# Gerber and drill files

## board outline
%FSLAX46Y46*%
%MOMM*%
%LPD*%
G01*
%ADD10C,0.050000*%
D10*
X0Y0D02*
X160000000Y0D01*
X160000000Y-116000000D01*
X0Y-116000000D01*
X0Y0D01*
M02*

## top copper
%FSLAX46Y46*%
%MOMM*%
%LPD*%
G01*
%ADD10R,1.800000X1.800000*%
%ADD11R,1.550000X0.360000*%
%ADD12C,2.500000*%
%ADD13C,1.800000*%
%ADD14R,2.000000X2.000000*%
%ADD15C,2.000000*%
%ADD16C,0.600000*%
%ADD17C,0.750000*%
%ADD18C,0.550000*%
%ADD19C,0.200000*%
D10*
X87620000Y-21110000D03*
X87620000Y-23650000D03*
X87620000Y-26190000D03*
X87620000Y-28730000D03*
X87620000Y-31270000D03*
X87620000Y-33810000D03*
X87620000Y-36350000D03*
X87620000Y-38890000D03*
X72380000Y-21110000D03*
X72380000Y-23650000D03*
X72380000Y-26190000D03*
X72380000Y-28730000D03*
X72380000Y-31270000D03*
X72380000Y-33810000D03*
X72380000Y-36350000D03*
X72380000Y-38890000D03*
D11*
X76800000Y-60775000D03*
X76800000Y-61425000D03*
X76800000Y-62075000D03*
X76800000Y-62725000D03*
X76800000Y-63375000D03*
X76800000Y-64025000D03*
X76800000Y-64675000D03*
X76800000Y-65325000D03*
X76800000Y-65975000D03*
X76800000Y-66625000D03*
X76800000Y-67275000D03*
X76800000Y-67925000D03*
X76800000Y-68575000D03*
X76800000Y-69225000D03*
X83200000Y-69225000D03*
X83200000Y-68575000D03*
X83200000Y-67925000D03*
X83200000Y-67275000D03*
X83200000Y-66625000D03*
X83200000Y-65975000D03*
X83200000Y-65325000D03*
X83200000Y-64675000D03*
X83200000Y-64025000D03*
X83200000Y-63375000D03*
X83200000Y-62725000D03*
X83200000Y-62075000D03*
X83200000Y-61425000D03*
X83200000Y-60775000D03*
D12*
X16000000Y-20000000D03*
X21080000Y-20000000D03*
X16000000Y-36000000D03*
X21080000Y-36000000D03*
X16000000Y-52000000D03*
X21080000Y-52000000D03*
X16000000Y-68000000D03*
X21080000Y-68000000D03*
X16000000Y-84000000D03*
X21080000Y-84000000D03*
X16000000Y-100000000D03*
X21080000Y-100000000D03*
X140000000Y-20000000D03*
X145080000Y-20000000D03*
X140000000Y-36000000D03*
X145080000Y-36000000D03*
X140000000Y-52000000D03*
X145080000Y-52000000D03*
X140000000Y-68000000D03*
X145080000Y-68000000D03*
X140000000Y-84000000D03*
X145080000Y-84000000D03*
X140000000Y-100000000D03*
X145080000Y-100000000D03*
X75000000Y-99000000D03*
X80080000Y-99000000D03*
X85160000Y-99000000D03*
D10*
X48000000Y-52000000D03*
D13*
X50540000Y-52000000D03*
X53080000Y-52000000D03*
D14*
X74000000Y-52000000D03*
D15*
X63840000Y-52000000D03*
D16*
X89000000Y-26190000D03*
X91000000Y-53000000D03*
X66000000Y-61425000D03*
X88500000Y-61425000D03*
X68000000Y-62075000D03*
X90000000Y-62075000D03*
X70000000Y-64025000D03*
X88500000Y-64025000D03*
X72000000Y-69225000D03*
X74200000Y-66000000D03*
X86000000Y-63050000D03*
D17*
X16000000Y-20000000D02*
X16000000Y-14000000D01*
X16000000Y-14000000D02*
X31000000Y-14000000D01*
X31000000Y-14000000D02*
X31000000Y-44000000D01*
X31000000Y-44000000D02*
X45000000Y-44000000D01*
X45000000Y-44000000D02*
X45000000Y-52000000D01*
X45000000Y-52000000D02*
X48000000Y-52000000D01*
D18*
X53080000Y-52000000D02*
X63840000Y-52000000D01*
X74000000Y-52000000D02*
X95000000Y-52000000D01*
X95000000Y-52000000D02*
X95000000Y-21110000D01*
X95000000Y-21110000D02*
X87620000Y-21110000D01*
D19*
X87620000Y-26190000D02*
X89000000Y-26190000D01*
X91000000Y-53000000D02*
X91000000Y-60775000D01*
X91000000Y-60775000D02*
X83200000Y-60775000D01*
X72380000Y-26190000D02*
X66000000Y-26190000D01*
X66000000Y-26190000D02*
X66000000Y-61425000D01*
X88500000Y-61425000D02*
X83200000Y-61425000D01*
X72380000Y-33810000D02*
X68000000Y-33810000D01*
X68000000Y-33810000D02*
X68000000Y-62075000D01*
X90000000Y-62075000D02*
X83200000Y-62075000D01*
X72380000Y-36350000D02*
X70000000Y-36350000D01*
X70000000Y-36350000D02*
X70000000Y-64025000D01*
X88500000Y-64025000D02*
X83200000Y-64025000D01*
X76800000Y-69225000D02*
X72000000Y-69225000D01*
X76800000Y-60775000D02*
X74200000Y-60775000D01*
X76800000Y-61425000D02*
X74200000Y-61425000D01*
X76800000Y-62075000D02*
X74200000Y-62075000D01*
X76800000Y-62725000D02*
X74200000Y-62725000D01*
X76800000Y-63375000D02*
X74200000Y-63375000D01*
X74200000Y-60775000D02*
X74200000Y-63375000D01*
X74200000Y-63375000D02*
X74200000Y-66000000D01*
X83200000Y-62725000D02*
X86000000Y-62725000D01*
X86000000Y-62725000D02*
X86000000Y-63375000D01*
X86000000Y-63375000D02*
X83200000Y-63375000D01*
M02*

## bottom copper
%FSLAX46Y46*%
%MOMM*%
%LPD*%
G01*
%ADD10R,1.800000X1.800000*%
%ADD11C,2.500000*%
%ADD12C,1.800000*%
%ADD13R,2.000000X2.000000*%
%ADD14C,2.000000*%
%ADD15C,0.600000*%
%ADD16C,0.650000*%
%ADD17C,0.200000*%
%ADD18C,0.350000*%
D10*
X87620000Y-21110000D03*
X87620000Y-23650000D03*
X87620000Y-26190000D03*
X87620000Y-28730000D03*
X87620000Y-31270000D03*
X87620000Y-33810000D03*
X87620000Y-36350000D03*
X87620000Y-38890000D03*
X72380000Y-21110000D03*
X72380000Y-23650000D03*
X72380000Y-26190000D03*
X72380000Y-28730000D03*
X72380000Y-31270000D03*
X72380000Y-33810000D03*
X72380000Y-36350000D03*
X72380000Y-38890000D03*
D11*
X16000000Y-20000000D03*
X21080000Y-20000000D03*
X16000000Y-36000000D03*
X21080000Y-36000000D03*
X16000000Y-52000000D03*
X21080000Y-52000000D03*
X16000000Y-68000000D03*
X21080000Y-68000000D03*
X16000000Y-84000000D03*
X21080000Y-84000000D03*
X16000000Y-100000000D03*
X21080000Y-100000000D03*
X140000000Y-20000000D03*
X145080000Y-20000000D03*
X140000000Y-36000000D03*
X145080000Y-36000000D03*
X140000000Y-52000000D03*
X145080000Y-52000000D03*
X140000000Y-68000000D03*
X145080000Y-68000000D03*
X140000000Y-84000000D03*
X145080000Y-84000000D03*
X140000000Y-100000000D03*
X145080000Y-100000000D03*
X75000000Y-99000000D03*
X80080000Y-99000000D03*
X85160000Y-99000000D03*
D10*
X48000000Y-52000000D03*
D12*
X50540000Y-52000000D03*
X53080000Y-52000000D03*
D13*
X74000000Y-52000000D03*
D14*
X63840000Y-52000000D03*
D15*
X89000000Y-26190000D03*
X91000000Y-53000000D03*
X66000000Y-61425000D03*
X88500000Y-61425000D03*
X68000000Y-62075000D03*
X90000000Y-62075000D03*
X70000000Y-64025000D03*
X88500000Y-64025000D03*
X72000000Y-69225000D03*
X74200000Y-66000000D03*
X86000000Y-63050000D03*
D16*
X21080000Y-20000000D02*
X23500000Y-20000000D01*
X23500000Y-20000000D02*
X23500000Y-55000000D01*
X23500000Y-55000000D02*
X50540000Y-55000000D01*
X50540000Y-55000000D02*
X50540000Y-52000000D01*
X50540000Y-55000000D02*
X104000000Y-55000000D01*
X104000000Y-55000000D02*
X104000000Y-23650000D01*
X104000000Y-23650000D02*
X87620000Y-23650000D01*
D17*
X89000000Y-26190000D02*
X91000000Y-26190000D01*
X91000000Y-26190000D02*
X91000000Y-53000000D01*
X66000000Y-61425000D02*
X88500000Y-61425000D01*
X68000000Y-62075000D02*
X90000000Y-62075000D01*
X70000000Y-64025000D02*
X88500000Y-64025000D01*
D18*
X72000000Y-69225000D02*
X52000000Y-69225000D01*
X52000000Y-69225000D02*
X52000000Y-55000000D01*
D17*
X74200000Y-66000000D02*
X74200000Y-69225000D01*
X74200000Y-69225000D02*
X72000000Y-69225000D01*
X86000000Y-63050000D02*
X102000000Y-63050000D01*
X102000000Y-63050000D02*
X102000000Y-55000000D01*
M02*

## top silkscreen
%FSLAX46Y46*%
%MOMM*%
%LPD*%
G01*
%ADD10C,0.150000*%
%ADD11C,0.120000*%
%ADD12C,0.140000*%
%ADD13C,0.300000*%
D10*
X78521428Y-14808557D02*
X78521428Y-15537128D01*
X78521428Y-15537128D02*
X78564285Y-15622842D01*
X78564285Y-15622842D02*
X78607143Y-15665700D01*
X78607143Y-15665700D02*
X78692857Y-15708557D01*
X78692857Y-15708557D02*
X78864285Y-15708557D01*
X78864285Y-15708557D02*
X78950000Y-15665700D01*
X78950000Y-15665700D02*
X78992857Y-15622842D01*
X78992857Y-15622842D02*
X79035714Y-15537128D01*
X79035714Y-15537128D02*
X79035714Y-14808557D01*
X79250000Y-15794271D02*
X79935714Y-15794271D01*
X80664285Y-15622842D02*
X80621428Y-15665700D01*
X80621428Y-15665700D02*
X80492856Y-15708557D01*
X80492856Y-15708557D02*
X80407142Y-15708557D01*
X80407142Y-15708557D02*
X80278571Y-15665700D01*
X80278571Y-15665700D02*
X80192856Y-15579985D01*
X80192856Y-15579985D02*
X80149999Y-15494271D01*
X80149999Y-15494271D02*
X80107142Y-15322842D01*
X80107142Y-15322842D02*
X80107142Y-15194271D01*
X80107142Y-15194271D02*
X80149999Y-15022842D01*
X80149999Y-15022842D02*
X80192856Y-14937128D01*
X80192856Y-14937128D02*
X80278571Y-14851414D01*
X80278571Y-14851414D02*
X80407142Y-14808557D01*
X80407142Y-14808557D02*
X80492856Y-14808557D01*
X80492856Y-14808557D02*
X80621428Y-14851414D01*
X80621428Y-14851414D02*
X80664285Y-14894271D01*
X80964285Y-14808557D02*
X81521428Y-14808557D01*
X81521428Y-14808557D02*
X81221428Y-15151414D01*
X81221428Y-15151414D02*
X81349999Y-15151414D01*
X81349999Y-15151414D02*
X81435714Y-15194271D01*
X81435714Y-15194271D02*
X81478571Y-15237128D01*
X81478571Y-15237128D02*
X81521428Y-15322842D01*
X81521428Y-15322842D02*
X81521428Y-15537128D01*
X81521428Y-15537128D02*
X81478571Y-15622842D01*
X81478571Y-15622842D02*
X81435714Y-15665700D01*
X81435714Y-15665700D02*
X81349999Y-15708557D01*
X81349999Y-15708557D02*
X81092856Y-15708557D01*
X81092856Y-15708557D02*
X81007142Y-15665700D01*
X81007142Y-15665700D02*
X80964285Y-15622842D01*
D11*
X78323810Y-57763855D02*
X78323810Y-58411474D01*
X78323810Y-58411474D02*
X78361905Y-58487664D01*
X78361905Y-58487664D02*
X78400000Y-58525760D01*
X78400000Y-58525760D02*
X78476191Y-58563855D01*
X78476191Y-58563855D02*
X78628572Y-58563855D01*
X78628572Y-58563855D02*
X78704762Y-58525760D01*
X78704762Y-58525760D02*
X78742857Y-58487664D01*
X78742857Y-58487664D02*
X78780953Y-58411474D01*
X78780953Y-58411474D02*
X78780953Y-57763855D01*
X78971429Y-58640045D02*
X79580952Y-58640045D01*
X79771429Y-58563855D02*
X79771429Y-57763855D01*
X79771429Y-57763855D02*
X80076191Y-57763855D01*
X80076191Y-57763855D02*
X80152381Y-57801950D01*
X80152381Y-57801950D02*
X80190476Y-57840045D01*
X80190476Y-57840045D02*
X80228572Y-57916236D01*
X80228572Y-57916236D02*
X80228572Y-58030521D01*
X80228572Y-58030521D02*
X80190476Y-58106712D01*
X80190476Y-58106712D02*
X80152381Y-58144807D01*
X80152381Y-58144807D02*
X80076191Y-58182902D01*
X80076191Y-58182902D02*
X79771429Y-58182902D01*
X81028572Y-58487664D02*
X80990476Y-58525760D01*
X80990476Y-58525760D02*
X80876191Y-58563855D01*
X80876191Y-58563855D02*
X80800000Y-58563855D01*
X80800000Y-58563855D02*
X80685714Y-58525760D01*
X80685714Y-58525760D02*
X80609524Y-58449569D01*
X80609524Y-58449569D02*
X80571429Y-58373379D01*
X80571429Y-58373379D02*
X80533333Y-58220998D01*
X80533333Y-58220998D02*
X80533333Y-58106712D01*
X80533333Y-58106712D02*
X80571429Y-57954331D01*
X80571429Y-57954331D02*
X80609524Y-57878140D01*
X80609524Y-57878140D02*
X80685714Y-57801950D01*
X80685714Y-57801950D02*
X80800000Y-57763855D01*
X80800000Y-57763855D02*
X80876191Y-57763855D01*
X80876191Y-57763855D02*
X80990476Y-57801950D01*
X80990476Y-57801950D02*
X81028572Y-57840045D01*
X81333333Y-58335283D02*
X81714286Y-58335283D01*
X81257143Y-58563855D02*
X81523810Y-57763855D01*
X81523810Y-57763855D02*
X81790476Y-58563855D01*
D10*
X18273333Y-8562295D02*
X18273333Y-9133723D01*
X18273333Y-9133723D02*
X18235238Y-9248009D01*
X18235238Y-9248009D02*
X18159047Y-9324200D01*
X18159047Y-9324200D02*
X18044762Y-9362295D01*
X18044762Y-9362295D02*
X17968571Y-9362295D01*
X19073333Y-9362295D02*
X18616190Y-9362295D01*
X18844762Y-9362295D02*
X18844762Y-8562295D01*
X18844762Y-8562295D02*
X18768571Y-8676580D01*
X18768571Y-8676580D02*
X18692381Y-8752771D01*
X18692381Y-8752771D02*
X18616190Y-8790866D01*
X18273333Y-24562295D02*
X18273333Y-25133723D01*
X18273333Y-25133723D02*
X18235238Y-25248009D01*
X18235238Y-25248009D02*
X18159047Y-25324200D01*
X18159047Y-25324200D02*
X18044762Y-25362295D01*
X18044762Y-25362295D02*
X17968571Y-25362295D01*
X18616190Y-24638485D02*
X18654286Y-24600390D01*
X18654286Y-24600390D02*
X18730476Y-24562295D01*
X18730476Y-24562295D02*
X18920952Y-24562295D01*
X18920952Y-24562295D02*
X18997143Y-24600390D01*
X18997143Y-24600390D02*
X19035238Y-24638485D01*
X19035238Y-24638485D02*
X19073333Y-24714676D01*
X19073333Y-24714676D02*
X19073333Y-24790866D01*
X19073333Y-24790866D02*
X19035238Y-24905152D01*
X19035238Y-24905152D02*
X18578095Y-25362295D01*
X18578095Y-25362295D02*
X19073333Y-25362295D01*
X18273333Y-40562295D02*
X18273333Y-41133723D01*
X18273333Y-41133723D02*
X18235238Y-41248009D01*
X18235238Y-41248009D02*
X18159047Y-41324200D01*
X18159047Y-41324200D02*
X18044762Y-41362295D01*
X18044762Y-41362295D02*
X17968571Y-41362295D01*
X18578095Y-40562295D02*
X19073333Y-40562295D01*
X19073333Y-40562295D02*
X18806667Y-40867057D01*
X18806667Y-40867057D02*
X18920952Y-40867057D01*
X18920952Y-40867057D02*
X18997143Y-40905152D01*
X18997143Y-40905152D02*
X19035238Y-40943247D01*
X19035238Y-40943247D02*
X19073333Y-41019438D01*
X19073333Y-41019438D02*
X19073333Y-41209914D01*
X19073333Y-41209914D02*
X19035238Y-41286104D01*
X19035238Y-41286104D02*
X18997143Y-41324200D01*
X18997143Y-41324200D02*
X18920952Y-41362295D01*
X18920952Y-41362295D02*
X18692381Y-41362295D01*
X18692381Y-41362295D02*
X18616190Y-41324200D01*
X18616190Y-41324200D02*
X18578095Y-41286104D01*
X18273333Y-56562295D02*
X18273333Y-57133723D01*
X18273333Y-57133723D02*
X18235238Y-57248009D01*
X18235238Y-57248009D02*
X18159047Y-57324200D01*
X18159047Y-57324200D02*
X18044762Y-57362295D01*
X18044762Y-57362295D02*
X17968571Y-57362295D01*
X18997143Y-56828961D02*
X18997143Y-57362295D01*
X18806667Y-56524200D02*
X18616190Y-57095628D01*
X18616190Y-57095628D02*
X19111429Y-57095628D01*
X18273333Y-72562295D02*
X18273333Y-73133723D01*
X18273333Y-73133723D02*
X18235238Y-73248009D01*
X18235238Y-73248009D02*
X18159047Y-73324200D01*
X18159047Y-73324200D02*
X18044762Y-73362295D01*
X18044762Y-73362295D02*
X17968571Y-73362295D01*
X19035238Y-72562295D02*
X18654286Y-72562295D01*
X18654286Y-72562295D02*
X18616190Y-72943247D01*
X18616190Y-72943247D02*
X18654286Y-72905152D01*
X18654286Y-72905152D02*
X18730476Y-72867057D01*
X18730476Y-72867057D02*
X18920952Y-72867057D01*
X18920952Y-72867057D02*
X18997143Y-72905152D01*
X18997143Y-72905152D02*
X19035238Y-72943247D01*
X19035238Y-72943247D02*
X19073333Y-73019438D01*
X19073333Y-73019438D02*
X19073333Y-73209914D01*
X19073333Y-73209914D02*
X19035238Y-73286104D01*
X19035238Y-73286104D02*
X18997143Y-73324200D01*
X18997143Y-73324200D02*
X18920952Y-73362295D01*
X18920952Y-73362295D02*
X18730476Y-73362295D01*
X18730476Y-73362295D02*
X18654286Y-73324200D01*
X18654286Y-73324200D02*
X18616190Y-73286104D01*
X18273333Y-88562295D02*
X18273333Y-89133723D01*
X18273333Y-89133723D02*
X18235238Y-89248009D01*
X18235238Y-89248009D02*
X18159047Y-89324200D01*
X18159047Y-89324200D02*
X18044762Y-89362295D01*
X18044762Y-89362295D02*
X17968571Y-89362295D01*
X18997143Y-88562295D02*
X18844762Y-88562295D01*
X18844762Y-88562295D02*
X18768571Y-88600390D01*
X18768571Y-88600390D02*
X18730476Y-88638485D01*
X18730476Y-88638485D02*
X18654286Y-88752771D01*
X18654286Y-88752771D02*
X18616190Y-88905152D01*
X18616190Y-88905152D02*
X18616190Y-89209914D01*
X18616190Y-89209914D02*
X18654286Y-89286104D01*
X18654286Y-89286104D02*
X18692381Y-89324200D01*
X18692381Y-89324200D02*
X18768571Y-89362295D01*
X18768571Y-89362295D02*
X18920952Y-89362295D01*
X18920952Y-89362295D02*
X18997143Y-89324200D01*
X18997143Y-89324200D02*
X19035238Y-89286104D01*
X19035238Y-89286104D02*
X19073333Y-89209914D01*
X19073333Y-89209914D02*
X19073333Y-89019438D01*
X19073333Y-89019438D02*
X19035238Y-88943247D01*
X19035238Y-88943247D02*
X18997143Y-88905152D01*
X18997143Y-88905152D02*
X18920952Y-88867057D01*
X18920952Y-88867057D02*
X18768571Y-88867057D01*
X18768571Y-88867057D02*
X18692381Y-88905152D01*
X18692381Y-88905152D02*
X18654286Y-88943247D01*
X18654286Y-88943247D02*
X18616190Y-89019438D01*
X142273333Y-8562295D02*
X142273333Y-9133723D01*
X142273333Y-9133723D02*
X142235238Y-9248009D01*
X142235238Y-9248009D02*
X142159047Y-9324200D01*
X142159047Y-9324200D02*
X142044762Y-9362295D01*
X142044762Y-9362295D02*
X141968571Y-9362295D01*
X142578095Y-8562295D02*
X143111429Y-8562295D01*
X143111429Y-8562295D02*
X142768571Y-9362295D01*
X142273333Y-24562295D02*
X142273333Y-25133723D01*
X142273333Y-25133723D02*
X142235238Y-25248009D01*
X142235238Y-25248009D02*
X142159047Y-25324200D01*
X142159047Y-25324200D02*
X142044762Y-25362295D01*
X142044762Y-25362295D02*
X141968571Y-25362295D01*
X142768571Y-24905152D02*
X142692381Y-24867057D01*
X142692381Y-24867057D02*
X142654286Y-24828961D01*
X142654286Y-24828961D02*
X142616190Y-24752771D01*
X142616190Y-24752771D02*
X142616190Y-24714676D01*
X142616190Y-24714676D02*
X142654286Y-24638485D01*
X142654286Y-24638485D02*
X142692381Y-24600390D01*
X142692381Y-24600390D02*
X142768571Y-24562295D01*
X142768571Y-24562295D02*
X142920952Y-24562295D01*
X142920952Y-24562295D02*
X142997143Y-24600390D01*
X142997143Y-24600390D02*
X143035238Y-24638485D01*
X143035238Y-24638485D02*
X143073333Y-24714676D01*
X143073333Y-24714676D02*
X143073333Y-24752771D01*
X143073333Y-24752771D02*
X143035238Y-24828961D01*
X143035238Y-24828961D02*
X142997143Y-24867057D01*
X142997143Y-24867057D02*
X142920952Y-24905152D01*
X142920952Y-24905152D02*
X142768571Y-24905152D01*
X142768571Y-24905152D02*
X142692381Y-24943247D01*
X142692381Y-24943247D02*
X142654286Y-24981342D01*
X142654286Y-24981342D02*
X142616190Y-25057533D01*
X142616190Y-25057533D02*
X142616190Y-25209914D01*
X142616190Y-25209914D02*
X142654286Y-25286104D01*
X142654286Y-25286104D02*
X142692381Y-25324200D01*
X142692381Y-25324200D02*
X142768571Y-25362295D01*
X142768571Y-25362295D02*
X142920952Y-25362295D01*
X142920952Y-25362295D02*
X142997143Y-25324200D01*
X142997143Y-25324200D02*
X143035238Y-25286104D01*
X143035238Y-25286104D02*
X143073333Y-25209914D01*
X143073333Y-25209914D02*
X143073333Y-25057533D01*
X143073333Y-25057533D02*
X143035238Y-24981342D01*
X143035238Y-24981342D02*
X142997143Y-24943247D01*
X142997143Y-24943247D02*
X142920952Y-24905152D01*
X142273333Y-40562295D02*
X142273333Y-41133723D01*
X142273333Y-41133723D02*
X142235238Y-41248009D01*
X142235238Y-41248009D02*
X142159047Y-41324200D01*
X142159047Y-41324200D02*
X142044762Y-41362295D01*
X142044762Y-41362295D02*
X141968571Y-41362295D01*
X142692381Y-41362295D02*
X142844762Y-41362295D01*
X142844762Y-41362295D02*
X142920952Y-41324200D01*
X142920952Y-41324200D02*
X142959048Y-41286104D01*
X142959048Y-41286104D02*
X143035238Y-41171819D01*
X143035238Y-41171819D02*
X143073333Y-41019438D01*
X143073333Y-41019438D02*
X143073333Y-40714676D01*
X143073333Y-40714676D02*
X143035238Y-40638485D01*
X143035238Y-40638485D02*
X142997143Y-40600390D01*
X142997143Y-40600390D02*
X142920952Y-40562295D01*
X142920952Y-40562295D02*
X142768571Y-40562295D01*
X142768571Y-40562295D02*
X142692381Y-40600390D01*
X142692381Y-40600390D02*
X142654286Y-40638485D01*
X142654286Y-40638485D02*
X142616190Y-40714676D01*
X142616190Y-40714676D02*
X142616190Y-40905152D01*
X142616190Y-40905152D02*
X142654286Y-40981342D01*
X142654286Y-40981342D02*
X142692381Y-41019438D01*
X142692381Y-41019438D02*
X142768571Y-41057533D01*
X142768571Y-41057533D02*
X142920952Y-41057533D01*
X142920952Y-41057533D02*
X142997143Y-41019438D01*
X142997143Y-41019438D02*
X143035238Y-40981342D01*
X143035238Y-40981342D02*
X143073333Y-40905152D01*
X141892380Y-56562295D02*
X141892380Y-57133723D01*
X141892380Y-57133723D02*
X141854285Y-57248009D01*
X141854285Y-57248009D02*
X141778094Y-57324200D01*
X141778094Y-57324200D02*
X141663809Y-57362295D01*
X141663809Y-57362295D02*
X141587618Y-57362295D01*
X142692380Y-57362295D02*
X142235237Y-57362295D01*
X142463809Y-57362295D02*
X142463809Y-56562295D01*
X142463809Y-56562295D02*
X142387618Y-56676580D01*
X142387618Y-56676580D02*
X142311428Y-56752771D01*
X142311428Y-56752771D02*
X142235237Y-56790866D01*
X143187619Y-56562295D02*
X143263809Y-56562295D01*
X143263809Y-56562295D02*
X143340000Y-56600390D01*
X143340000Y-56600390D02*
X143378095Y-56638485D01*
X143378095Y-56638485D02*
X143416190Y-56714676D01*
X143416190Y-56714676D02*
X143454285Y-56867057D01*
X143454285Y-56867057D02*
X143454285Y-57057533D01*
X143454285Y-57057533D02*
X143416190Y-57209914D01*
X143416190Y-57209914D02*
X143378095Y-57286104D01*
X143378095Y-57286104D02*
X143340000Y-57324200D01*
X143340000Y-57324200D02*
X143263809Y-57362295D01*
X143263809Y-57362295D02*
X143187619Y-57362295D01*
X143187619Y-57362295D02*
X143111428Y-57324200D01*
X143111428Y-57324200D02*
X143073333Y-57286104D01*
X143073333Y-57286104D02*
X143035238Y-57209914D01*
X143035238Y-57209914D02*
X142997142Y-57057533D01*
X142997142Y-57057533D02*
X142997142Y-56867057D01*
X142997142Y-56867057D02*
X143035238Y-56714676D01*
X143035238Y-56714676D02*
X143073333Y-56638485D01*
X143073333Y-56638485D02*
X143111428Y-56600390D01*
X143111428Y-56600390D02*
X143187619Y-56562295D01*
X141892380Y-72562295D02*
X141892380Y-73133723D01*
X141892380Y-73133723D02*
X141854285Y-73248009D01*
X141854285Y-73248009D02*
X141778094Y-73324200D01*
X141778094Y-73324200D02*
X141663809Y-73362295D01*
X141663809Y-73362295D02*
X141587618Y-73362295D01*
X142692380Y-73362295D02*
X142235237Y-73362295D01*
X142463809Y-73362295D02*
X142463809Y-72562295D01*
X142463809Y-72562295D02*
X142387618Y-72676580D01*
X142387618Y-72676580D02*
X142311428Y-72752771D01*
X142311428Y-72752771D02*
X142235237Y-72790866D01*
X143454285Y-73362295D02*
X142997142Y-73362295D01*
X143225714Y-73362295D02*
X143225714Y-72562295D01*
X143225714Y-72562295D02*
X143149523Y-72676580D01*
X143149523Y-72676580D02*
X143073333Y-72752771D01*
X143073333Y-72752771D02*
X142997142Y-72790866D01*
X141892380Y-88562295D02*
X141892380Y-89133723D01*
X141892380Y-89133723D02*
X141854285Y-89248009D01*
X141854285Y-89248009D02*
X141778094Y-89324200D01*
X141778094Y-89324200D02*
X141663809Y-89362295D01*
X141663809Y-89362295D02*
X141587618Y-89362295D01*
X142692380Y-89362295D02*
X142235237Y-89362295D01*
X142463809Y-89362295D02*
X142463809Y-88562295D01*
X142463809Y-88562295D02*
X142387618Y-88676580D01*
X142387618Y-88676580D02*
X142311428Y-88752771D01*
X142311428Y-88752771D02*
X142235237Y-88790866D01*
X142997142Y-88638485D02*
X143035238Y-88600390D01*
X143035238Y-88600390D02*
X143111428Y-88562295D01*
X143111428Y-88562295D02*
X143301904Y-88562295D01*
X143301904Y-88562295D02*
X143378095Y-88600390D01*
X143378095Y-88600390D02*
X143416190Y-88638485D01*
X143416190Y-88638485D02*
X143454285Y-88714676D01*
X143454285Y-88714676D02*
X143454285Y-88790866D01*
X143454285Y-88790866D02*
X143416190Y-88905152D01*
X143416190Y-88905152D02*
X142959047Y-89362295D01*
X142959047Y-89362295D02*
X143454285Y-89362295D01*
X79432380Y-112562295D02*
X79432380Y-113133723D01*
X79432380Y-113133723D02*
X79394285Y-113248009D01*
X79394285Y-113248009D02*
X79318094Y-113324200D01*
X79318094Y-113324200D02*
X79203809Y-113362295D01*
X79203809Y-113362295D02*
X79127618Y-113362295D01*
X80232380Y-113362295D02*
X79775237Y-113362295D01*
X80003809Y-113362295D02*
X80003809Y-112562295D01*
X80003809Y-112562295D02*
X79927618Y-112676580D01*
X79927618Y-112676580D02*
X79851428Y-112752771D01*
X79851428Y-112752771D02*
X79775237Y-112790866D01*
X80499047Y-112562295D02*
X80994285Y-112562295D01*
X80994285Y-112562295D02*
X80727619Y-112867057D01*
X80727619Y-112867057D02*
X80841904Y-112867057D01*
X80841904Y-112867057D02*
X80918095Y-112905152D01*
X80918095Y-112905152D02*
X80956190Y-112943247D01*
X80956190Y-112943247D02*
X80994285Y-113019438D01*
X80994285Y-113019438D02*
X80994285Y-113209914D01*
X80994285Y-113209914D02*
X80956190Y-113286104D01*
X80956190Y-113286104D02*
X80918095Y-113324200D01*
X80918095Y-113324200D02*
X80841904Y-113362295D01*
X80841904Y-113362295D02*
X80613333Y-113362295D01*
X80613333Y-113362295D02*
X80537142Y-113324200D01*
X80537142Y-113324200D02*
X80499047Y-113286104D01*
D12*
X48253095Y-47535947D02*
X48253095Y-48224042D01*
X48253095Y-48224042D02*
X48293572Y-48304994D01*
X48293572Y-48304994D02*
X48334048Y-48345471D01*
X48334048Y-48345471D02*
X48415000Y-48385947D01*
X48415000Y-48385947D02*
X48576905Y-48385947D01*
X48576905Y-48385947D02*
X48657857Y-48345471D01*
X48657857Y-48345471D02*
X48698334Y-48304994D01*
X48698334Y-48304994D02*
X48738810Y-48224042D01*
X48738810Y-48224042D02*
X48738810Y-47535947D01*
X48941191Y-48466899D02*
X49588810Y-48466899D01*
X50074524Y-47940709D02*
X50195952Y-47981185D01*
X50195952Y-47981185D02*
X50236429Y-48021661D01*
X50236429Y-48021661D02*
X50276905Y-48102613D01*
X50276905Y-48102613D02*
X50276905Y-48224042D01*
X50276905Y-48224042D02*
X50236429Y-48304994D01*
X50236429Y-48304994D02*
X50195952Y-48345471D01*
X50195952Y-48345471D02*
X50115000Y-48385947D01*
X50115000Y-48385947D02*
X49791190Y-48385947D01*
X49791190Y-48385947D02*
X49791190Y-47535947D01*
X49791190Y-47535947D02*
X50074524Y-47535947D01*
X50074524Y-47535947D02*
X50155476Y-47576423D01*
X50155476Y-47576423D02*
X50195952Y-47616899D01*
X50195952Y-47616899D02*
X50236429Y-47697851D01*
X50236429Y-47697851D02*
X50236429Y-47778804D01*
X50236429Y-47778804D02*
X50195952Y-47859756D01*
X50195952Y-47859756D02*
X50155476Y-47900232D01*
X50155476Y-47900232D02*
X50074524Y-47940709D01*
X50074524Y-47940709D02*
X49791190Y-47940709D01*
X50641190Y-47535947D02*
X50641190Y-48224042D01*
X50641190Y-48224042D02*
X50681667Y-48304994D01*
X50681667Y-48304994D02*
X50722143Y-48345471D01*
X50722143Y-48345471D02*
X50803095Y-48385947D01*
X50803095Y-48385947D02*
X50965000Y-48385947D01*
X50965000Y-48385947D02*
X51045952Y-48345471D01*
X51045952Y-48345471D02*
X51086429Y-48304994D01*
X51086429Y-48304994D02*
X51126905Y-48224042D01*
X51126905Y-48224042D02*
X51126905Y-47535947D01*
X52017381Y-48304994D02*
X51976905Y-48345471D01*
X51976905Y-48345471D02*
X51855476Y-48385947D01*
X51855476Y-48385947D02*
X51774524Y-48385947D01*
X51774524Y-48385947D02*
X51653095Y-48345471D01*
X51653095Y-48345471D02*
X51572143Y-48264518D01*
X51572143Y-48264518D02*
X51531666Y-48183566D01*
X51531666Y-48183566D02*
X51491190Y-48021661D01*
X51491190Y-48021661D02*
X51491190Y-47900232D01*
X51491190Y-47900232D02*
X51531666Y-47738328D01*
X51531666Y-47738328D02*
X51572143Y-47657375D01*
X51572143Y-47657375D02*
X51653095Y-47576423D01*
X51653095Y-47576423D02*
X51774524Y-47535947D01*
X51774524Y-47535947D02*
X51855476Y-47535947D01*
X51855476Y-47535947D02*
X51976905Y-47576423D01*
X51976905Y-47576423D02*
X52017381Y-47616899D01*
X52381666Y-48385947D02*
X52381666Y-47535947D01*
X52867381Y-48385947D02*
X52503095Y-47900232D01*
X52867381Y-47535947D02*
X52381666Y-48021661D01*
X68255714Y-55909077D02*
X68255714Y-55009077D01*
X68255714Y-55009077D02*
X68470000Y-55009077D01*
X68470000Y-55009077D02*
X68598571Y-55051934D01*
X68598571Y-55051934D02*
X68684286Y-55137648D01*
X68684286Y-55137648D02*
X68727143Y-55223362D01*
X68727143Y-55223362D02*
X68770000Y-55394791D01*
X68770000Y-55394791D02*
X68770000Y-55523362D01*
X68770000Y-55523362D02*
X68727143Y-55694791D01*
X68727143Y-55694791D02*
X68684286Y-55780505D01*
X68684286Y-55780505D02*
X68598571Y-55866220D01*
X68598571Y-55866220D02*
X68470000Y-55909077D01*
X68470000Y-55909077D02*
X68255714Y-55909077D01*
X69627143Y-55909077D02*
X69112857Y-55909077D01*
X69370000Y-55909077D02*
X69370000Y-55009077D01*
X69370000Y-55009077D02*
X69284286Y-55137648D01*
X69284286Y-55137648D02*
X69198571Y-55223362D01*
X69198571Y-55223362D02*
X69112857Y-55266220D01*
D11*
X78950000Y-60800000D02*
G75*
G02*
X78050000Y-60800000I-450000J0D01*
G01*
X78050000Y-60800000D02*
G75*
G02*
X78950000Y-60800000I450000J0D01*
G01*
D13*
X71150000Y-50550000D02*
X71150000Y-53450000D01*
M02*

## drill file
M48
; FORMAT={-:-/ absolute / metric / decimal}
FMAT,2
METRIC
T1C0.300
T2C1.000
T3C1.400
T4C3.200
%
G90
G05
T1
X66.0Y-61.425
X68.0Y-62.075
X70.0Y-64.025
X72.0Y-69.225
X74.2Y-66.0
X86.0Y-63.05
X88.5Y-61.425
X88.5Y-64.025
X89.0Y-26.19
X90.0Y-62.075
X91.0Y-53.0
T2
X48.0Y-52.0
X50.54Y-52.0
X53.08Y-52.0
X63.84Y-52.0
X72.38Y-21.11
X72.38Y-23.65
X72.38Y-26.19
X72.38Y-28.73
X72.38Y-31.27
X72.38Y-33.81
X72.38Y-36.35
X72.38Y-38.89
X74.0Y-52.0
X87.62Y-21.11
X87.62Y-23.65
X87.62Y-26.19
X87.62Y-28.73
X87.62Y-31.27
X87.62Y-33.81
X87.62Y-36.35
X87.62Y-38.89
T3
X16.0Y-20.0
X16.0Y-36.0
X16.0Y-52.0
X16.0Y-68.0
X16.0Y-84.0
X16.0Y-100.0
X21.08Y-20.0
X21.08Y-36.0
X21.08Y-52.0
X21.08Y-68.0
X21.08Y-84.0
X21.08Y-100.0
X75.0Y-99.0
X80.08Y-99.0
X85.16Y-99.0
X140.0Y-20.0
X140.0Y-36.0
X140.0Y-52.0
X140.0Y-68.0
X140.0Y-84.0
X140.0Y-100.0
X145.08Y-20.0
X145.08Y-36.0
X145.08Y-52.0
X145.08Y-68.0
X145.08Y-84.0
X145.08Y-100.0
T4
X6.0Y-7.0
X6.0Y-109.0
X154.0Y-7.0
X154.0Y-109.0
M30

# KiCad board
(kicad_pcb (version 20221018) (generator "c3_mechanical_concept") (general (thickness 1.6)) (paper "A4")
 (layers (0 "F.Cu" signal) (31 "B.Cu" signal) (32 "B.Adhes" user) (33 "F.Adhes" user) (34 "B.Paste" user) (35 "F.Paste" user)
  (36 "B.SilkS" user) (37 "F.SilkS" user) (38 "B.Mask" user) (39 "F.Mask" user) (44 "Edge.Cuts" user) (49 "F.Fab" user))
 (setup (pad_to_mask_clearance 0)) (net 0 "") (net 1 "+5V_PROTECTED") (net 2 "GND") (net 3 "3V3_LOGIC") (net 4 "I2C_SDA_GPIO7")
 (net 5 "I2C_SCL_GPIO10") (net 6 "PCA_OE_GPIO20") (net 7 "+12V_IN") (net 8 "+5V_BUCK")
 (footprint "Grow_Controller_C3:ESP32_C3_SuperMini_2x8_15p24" (layer "F.Cu") (at 80 30)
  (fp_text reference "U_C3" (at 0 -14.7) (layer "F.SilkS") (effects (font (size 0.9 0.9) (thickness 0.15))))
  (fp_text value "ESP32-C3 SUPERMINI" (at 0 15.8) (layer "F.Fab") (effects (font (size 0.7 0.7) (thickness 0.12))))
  (pad "1" thru_hole rect (at 7.62 -8.89) (size 1.8 1.8) (drill 1.0) (layers "*.Cu" "*.Mask") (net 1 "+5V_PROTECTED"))
  (pad "2" thru_hole rect (at 7.62 -6.35) (size 1.8 1.8) (drill 1.0) (layers "*.Cu" "*.Mask") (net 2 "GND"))
  (pad "3" thru_hole rect (at 7.62 -3.81) (size 1.8 1.8) (drill 1.0) (layers "*.Cu" "*.Mask") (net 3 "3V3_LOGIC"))
  (pad "4" thru_hole rect (at 7.62 -1.27) (size 1.8 1.8) (drill 1.0) (layers "*.Cu" "*.Mask"))
  (pad "5" thru_hole rect (at 7.62 1.27) (size 1.8 1.8) (drill 1.0) (layers "*.Cu" "*.Mask"))
  (pad "6" thru_hole rect (at 7.62 3.81) (size 1.8 1.8) (drill 1.0) (layers "*.Cu" "*.Mask"))
  (pad "7" thru_hole rect (at 7.62 6.35) (size 1.8 1.8) (drill 1.0) (layers "*.Cu" "*.Mask"))
  (pad "8" thru_hole rect (at 7.62 8.89) (size 1.8 1.8) (drill 1.0) (layers "*.Cu" "*.Mask"))
  (pad "9" thru_hole rect (at -7.62 -8.89) (size 1.8 1.8) (drill 1.0) (layers "*.Cu" "*.Mask"))
  (pad "10" thru_hole rect (at -7.62 -6.35) (size 1.8 1.8) (drill 1.0) (layers "*.Cu" "*.Mask"))
  (pad "11" thru_hole rect (at -7.62 -3.81) (size 1.8 1.8) (drill 1.0) (layers "*.Cu" "*.Mask") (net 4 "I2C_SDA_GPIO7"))
  (pad "12" thru_hole rect (at -7.62 -1.27) (size 1.8 1.8) (drill 1.0) (layers "*.Cu" "*.Mask"))
  (pad "13" thru_hole rect (at -7.62 1.27) (size 1.8 1.8) (drill 1.0) (layers "*.Cu" "*.Mask"))
  (pad "14" thru_hole rect (at -7.62 3.81) (size 1.8 1.8) (drill 1.0) (layers "*.Cu" "*.Mask") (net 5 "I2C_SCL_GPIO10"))
  (pad "15" thru_hole rect (at -7.62 6.35) (size 1.8 1.8) (drill 1.0) (layers "*.Cu" "*.Mask") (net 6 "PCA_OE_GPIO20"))
  (pad "16" thru_hole rect (at -7.62 8.89) (size 1.8 1.8) (drill 1.0) (layers "*.Cu" "*.Mask")))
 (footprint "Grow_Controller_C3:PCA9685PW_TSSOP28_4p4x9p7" (layer "F.Cu") (at 80 65)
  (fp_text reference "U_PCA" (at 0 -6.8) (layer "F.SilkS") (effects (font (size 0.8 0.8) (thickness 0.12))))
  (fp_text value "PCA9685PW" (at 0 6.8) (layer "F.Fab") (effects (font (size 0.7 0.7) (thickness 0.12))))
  (fp_circle (center -1.5 -4.2) (end -1.05 -4.2) (stroke (width 0.12) (type solid)) (fill none) (layer "F.SilkS"))
  (pad "1" smd rect (at -3.200 -4.225) (size 1.55 0.36) (layers "F.Cu" "F.Paste" "F.Mask") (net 2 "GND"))
  (pad "2" smd rect (at -3.200 -3.575) (size 1.55 0.36) (layers "F.Cu" "F.Paste" "F.Mask") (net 2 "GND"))
  (pad "3" smd rect (at -3.200 -2.925) (size 1.55 0.36) (layers "F.Cu" "F.Paste" "F.Mask") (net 2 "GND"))
  (pad "4" smd rect (at -3.200 -2.275) (size 1.55 0.36) (layers "F.Cu" "F.Paste" "F.Mask") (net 2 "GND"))
  (pad "5" smd rect (at -3.200 -1.625) (size 1.55 0.36) (layers "F.Cu" "F.Paste" "F.Mask") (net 2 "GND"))
  (pad "6" smd rect (at -3.200 -0.975) (size 1.55 0.36) (layers "F.Cu" "F.Paste" "F.Mask"))
  (pad "7" smd rect (at -3.200 -0.325) (size 1.55 0.36) (layers "F.Cu" "F.Paste" "F.Mask"))
  (pad "8" smd rect (at -3.200 0.325) (size 1.55 0.36) (layers "F.Cu" "F.Paste" "F.Mask"))
  (pad "9" smd rect (at -3.200 0.975) (size 1.55 0.36) (layers "F.Cu" "F.Paste" "F.Mask"))
  (pad "10" smd rect (at -3.200 1.625) (size 1.55 0.36) (layers "F.Cu" "F.Paste" "F.Mask"))
  (pad "11" smd rect (at -3.200 2.275) (size 1.55 0.36) (layers "F.Cu" "F.Paste" "F.Mask"))
  (pad "12" smd rect (at -3.200 2.925) (size 1.55 0.36) (layers "F.Cu" "F.Paste" "F.Mask"))
  (pad "13" smd rect (at -3.200 3.575) (size 1.55 0.36) (layers "F.Cu" "F.Paste" "F.Mask"))
  (pad "14" smd rect (at -3.200 4.225) (size 1.55 0.36) (layers "F.Cu" "F.Paste" "F.Mask") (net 2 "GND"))
  (pad "15" smd rect (at 3.200 4.225) (size 1.55 0.36) (layers "F.Cu" "F.Paste" "F.Mask"))
  (pad "16" smd rect (at 3.200 3.575) (size 1.55 0.36) (layers "F.Cu" "F.Paste" "F.Mask"))
  (pad "17" smd rect (at 3.200 2.925) (size 1.55 0.36) (layers "F.Cu" "F.Paste" "F.Mask"))
  (pad "18" smd rect (at 3.200 2.275) (size 1.55 0.36) (layers "F.Cu" "F.Paste" "F.Mask"))
  (pad "19" smd rect (at 3.200 1.625) (size 1.55 0.36) (layers "F.Cu" "F.Paste" "F.Mask"))
  (pad "20" smd rect (at 3.200 0.975) (size 1.55 0.36) (layers "F.Cu" "F.Paste" "F.Mask"))
  (pad "21" smd rect (at 3.200 0.325) (size 1.55 0.36) (layers "F.Cu" "F.Paste" "F.Mask"))
  (pad "22" smd rect (at 3.200 -0.325) (size 1.55 0.36) (layers "F.Cu" "F.Paste" "F.Mask"))
  (pad "23" smd rect (at 3.200 -0.975) (size 1.55 0.36) (layers "F.Cu" "F.Paste" "F.Mask") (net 6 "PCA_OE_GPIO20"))
  (pad "24" smd rect (at 3.200 -1.625) (size 1.55 0.36) (layers "F.Cu" "F.Paste" "F.Mask") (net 2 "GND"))
  (pad "25" smd rect (at 3.200 -2.275) (size 1.55 0.36) (layers "F.Cu" "F.Paste" "F.Mask") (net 2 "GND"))
  (pad "26" smd rect (at 3.200 -2.925) (size 1.55 0.36) (layers "F.Cu" "F.Paste" "F.Mask") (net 5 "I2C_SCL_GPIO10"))
  (pad "27" smd rect (at 3.200 -3.575) (size 1.55 0.36) (layers "F.Cu" "F.Paste" "F.Mask") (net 4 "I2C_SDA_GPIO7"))
  (pad "28" smd rect (at 3.200 -4.225) (size 1.55 0.36) (layers "F.Cu" "F.Paste" "F.Mask") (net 3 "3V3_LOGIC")))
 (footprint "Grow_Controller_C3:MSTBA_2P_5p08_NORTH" (layer "F.Cu") (at 16 20)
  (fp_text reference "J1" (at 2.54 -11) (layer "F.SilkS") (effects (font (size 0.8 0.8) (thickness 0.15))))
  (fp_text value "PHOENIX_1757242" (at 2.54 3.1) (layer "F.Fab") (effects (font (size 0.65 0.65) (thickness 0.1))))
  (pad "1" thru_hole circle (at 0.00 0) (size 2.5 2.5) (drill 1.4) (layers "*.Cu" "*.Mask") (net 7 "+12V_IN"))
  (pad "2" thru_hole circle (at 5.08 0) (size 2.5 2.5) (drill 1.4) (layers "*.Cu" "*.Mask") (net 2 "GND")))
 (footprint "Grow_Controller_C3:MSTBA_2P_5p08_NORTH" (layer "F.Cu") (at 16 36)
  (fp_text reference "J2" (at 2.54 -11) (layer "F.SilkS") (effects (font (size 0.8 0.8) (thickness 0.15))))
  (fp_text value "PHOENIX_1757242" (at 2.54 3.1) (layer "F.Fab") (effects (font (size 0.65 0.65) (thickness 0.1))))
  (pad "1" thru_hole circle (at 0.00 0) (size 2.5 2.5) (drill 1.4) (layers "*.Cu" "*.Mask"))
  (pad "2" thru_hole circle (at 5.08 0) (size 2.5 2.5) (drill 1.4) (layers "*.Cu" "*.Mask")))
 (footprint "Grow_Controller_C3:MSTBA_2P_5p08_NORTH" (layer "F.Cu") (at 16 52)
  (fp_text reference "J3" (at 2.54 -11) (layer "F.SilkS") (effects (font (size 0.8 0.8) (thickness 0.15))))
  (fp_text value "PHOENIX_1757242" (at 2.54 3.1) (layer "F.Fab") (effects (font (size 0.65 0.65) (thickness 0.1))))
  (pad "1" thru_hole circle (at 0.00 0) (size 2.5 2.5) (drill 1.4) (layers "*.Cu" "*.Mask"))
  (pad "2" thru_hole circle (at 5.08 0) (size 2.5 2.5) (drill 1.4) (layers "*.Cu" "*.Mask")))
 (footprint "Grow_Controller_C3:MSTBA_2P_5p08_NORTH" (layer "F.Cu") (at 16 68)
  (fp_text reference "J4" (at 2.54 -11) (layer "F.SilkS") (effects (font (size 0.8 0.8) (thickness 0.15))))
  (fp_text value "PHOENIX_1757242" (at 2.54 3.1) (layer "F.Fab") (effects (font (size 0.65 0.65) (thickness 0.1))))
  (pad "1" thru_hole circle (at 0.00 0) (size 2.5 2.5) (drill 1.4) (layers "*.Cu" "*.Mask"))
  (pad "2" thru_hole circle (at 5.08 0) (size 2.5 2.5) (drill 1.4) (layers "*.Cu" "*.Mask")))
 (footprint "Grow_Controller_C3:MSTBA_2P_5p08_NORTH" (layer "F.Cu") (at 16 84)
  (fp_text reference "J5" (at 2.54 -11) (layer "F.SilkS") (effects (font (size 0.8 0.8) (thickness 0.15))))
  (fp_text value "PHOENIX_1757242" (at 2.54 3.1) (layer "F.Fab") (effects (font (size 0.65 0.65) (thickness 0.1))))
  (pad "1" thru_hole circle (at 0.00 0) (size 2.5 2.5) (drill 1.4) (layers "*.Cu" "*.Mask"))
  (pad "2" thru_hole circle (at 5.08 0) (size 2.5 2.5) (drill 1.4) (layers "*.Cu" "*.Mask")))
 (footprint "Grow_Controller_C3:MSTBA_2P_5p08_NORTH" (layer "F.Cu") (at 16 100)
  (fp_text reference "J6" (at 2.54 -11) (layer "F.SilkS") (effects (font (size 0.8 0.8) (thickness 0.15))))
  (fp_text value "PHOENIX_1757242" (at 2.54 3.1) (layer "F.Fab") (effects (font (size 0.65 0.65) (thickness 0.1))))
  (pad "1" thru_hole circle (at 0.00 0) (size 2.5 2.5) (drill 1.4) (layers "*.Cu" "*.Mask"))
  (pad "2" thru_hole circle (at 5.08 0) (size 2.5 2.5) (drill 1.4) (layers "*.Cu" "*.Mask")))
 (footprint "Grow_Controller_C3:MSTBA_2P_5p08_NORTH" (layer "F.Cu") (at 140 20)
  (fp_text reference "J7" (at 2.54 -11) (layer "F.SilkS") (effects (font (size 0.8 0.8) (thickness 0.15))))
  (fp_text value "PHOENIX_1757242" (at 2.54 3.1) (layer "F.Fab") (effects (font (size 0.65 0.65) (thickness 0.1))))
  (pad "1" thru_hole circle (at 0.00 0) (size 2.5 2.5) (drill 1.4) (layers "*.Cu" "*.Mask"))
  (pad "2" thru_hole circle (at 5.08 0) (size 2.5 2.5) (drill 1.4) (layers "*.Cu" "*.Mask")))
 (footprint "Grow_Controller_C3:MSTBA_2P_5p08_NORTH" (layer "F.Cu") (at 140 36)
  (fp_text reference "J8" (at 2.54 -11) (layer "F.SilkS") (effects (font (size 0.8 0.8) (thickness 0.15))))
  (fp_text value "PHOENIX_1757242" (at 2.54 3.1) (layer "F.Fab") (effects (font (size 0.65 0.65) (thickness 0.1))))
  (pad "1" thru_hole circle (at 0.00 0) (size 2.5 2.5) (drill 1.4) (layers "*.Cu" "*.Mask"))
  (pad "2" thru_hole circle (at 5.08 0) (size 2.5 2.5) (drill 1.4) (layers "*.Cu" "*.Mask")))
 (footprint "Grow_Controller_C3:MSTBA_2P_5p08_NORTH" (layer "F.Cu") (at 140 52)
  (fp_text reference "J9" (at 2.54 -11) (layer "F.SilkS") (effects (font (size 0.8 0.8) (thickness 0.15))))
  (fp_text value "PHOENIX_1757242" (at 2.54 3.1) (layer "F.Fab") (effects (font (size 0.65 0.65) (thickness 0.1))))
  (pad "1" thru_hole circle (at 0.00 0) (size 2.5 2.5) (drill 1.4) (layers "*.Cu" "*.Mask"))
  (pad "2" thru_hole circle (at 5.08 0) (size 2.5 2.5) (drill 1.4) (layers "*.Cu" "*.Mask")))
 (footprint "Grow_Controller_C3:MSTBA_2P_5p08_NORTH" (layer "F.Cu") (at 140 68)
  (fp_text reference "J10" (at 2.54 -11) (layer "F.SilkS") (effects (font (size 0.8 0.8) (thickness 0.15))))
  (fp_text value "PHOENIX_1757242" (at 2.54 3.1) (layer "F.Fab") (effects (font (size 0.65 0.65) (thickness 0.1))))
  (pad "1" thru_hole circle (at 0.00 0) (size 2.5 2.5) (drill 1.4) (layers "*.Cu" "*.Mask"))
  (pad "2" thru_hole circle (at 5.08 0) (size 2.5 2.5) (drill 1.4) (layers "*.Cu" "*.Mask")))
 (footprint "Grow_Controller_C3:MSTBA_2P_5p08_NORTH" (layer "F.Cu") (at 140 84)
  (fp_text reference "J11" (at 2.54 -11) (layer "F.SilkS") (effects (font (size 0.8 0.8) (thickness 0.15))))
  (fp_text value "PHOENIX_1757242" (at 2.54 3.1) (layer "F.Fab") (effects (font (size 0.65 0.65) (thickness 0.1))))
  (pad "1" thru_hole circle (at 0.00 0) (size 2.5 2.5) (drill 1.4) (layers "*.Cu" "*.Mask"))
  (pad "2" thru_hole circle (at 5.08 0) (size 2.5 2.5) (drill 1.4) (layers "*.Cu" "*.Mask")))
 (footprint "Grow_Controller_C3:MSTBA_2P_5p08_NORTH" (layer "F.Cu") (at 140 100)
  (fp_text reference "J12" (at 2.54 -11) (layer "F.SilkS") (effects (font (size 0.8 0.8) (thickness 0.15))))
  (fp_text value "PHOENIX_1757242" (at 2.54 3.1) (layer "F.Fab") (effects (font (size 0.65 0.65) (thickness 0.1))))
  (pad "1" thru_hole circle (at 0.00 0) (size 2.5 2.5) (drill 1.4) (layers "*.Cu" "*.Mask"))
  (pad "2" thru_hole circle (at 5.08 0) (size 2.5 2.5) (drill 1.4) (layers "*.Cu" "*.Mask")))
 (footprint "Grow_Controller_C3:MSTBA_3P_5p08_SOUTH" (layer "F.Cu") (at 75 99)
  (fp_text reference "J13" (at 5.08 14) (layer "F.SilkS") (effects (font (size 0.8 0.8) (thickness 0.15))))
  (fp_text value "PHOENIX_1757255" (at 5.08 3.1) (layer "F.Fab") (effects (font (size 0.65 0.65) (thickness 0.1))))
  (pad "1" thru_hole circle (at 0.00 0) (size 2.5 2.5) (drill 1.4) (layers "*.Cu" "*.Mask"))
  (pad "2" thru_hole circle (at 5.08 0) (size 2.5 2.5) (drill 1.4) (layers "*.Cu" "*.Mask"))
  (pad "3" thru_hole circle (at 10.16 0) (size 2.5 2.5) (drill 1.4) (layers "*.Cu" "*.Mask")))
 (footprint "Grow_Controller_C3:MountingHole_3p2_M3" (layer "F.Cu") (at 6 7)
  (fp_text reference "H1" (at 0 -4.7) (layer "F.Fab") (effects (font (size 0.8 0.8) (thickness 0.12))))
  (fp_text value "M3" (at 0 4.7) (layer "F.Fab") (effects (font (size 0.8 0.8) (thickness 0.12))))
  (pad "" np_thru_hole circle (at 0 0) (size 3.2 3.2) (drill 3.2) (layers "*.Cu" "*.Mask")))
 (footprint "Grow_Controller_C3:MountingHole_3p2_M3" (layer "F.Cu") (at 154 7)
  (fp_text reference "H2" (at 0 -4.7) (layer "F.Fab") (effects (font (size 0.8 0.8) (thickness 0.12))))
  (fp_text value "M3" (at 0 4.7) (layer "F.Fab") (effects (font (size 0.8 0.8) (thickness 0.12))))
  (pad "" np_thru_hole circle (at 0 0) (size 3.2 3.2) (drill 3.2) (layers "*.Cu" "*.Mask")))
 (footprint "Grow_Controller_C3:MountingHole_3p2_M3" (layer "F.Cu") (at 6 109)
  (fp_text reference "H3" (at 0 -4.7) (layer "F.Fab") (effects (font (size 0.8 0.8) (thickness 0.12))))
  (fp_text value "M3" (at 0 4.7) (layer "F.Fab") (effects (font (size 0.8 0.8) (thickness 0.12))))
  (pad "" np_thru_hole circle (at 0 0) (size 3.2 3.2) (drill 3.2) (layers "*.Cu" "*.Mask")))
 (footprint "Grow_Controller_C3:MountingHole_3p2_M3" (layer "F.Cu") (at 154 109)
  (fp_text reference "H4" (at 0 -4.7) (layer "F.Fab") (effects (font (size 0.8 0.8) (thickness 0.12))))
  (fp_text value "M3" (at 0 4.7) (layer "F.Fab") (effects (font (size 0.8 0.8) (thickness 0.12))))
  (pad "" np_thru_hole circle (at 0 0) (size 3.2 3.2) (drill 3.2) (layers "*.Cu" "*.Mask")))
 (gr_rect (start 0 0) (end 160 116) (stroke (width 0.05) (type default)) (fill none) (layer "Edge.Cuts"))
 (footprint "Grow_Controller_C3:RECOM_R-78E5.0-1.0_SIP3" (layer "F.Cu") (at 48 52)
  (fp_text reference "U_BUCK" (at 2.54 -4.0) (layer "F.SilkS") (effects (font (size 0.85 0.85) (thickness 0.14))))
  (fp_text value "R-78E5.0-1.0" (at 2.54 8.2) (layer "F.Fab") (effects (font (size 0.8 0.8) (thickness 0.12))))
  (pad "1" thru_hole rect (at 0 0) (size 1.8 1.8) (drill 1.0) (layers "*.Cu" "*.Mask") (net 7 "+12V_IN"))
  (pad "2" thru_hole circle (at 2.54 0) (size 1.8 1.8) (drill 1.0) (layers "*.Cu" "*.Mask") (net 2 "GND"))
  (pad "3" thru_hole circle (at 5.08 0) (size 1.8 1.8) (drill 1.0) (layers "*.Cu" "*.Mask") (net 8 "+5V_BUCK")))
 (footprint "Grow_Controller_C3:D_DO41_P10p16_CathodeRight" (layer "F.Cu") (at 63.84 52)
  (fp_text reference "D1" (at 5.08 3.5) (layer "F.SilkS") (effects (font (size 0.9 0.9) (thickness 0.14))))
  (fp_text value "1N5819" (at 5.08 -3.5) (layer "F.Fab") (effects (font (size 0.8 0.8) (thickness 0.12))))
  (fp_line (start 7.31 -1.45) (end 7.31 1.45) (stroke (width 0.3) (type solid)) (layer "F.SilkS"))
  (pad "1" thru_hole rect (at 10.16 0) (size 2.0 2.0) (drill 1.0) (layers "*.Cu" "*.Mask") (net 1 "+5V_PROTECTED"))
  (pad "2" thru_hole circle (at 0 0) (size 2.0 2.0) (drill 1.0) (layers "*.Cu" "*.Mask") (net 8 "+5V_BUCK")))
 (segment (start 16 20) (end 16 14) (width 0.75) (layer "F.Cu") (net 7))
 (segment (start 16 14) (end 31 14) (width 0.75) (layer "F.Cu") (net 7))
 (segment (start 31 14) (end 31 44) (width 0.75) (layer "F.Cu") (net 7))
 (segment (start 31 44) (end 45 44) (width 0.75) (layer "F.Cu") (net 7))
 (segment (start 45 44) (end 45 52) (width 0.75) (layer "F.Cu") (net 7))
 (segment (start 45 52) (end 48 52) (width 0.75) (layer "F.Cu") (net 7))
 (segment (start 21.08 20) (end 23.5 20) (width 0.65) (layer "B.Cu") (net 2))
 (segment (start 23.5 20) (end 23.5 55) (width 0.65) (layer "B.Cu") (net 2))
 (segment (start 23.5 55) (end 50.54 55) (width 0.65) (layer "B.Cu") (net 2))
 (segment (start 50.54 55) (end 50.54 52) (width 0.65) (layer "B.Cu") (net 2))
 (segment (start 50.54 55) (end 104 55) (width 0.65) (layer "B.Cu") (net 2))
 (segment (start 104 55) (end 104 23.65) (width 0.65) (layer "B.Cu") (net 2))
 (segment (start 104 23.65) (end 87.62 23.65) (width 0.65) (layer "B.Cu") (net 2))
 (segment (start 53.08 52) (end 63.84 52) (width 0.55) (layer "F.Cu") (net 8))
 (segment (start 74 52) (end 95 52) (width 0.55) (layer "F.Cu") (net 1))
 (segment (start 95 52) (end 95 21.11) (width 0.55) (layer "F.Cu") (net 1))
 (segment (start 95 21.11) (end 87.62 21.11) (width 0.55) (layer "F.Cu") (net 1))
 (segment (start 87.62 26.19) (end 89 26.19) (width 0.2) (layer "F.Cu") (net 3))
 (via (at 89 26.19) (size 0.6) (drill 0.3) (layers "F.Cu" "B.Cu") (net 3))
 (segment (start 89 26.19) (end 91 26.19) (width 0.2) (layer "B.Cu") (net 3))
 (segment (start 91 26.19) (end 91 53) (width 0.2) (layer "B.Cu") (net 3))
 (via (at 91 53) (size 0.6) (drill 0.3) (layers "F.Cu" "B.Cu") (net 3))
 (segment (start 91 53) (end 91 60.775) (width 0.2) (layer "F.Cu") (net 3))
 (segment (start 91 60.775) (end 83.2 60.775) (width 0.2) (layer "F.Cu") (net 3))
 (segment (start 72.38 26.19) (end 66 26.19) (width 0.2) (layer "F.Cu") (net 4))
 (segment (start 66 26.19) (end 66 61.425) (width 0.2) (layer "F.Cu") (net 4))
 (via (at 66 61.425) (size 0.6) (drill 0.3) (layers "F.Cu" "B.Cu") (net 4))
 (segment (start 66 61.425) (end 88.5 61.425) (width 0.2) (layer "B.Cu") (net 4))
 (via (at 88.5 61.425) (size 0.6) (drill 0.3) (layers "F.Cu" "B.Cu") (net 4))
 (segment (start 88.5 61.425) (end 83.2 61.425) (width 0.2) (layer "F.Cu") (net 4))
 (segment (start 72.38 33.81) (end 68 33.81) (width 0.2) (layer "F.Cu") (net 5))
 (segment (start 68 33.81) (end 68 62.075) (width 0.2) (layer "F.Cu") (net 5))
 (via (at 68 62.075) (size 0.6) (drill 0.3) (layers "F.Cu" "B.Cu") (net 5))
 (segment (start 68 62.075) (end 90 62.075) (width 0.2) (layer "B.Cu") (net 5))
 (via (at 90 62.075) (size 0.6) (drill 0.3) (layers "F.Cu" "B.Cu") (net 5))
 (segment (start 90 62.075) (end 83.2 62.075) (width 0.2) (layer "F.Cu") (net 5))
 (segment (start 72.38 36.35) (end 70 36.35) (width 0.2) (layer "F.Cu") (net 6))
 (segment (start 70 36.35) (end 70 64.025) (width 0.2) (layer "F.Cu") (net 6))
 (via (at 70 64.025) (size 0.6) (drill 0.3) (layers "F.Cu" "B.Cu") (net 6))
 (segment (start 70 64.025) (end 88.5 64.025) (width 0.2) (layer "B.Cu") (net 6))
 (via (at 88.5 64.025) (size 0.6) (drill 0.3) (layers "F.Cu" "B.Cu") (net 6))
 (segment (start 88.5 64.025) (end 83.2 64.025) (width 0.2) (layer "F.Cu") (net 6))
 (segment (start 76.8 69.225) (end 72 69.225) (width 0.2) (layer "F.Cu") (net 2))
 (via (at 72 69.225) (size 0.6) (drill 0.3) (layers "F.Cu" "B.Cu") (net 2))
 (segment (start 72 69.225) (end 52 69.225) (width 0.35) (layer "B.Cu") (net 2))
 (segment (start 52 69.225) (end 52 55) (width 0.35) (layer "B.Cu") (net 2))
 (segment (start 76.8 60.775) (end 74.2 60.775) (width 0.2) (layer "F.Cu") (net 2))
 (segment (start 76.8 61.425) (end 74.2 61.425) (width 0.2) (layer "F.Cu") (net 2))
 (segment (start 76.8 62.075) (end 74.2 62.075) (width 0.2) (layer "F.Cu") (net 2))
 (segment (start 76.8 62.725) (end 74.2 62.725) (width 0.2) (layer "F.Cu") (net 2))
 (segment (start 76.8 63.375) (end 74.2 63.375) (width 0.2) (layer "F.Cu") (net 2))
 (segment (start 74.2 60.775) (end 74.2 63.375) (width 0.2) (layer "F.Cu") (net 2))
 (segment (start 74.2 63.375) (end 74.2 66) (width 0.2) (layer "F.Cu") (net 2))
 (via (at 74.2 66) (size 0.6) (drill 0.3) (layers "F.Cu" "B.Cu") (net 2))
 (segment (start 74.2 66) (end 74.2 69.225) (width 0.2) (layer "B.Cu") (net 2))
 (segment (start 74.2 69.225) (end 72 69.225) (width 0.2) (layer "B.Cu") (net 2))
 (segment (start 83.2 62.725) (end 86 62.725) (width 0.2) (layer "F.Cu") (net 2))
 (segment (start 86 62.725) (end 86 63.375) (width 0.2) (layer "F.Cu") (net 2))
 (segment (start 86 63.375) (end 83.2 63.375) (width 0.2) (layer "F.Cu") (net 2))
 (via (at 86 63.05) (size 0.6) (drill 0.3) (layers "F.Cu" "B.Cu") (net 2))
 (segment (start 86 63.05) (end 102 63.05) (width 0.2) (layer "B.Cu") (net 2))
 (segment (start 102 63.05) (end 102 55) (width 0.2) (layer "B.Cu") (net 2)))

